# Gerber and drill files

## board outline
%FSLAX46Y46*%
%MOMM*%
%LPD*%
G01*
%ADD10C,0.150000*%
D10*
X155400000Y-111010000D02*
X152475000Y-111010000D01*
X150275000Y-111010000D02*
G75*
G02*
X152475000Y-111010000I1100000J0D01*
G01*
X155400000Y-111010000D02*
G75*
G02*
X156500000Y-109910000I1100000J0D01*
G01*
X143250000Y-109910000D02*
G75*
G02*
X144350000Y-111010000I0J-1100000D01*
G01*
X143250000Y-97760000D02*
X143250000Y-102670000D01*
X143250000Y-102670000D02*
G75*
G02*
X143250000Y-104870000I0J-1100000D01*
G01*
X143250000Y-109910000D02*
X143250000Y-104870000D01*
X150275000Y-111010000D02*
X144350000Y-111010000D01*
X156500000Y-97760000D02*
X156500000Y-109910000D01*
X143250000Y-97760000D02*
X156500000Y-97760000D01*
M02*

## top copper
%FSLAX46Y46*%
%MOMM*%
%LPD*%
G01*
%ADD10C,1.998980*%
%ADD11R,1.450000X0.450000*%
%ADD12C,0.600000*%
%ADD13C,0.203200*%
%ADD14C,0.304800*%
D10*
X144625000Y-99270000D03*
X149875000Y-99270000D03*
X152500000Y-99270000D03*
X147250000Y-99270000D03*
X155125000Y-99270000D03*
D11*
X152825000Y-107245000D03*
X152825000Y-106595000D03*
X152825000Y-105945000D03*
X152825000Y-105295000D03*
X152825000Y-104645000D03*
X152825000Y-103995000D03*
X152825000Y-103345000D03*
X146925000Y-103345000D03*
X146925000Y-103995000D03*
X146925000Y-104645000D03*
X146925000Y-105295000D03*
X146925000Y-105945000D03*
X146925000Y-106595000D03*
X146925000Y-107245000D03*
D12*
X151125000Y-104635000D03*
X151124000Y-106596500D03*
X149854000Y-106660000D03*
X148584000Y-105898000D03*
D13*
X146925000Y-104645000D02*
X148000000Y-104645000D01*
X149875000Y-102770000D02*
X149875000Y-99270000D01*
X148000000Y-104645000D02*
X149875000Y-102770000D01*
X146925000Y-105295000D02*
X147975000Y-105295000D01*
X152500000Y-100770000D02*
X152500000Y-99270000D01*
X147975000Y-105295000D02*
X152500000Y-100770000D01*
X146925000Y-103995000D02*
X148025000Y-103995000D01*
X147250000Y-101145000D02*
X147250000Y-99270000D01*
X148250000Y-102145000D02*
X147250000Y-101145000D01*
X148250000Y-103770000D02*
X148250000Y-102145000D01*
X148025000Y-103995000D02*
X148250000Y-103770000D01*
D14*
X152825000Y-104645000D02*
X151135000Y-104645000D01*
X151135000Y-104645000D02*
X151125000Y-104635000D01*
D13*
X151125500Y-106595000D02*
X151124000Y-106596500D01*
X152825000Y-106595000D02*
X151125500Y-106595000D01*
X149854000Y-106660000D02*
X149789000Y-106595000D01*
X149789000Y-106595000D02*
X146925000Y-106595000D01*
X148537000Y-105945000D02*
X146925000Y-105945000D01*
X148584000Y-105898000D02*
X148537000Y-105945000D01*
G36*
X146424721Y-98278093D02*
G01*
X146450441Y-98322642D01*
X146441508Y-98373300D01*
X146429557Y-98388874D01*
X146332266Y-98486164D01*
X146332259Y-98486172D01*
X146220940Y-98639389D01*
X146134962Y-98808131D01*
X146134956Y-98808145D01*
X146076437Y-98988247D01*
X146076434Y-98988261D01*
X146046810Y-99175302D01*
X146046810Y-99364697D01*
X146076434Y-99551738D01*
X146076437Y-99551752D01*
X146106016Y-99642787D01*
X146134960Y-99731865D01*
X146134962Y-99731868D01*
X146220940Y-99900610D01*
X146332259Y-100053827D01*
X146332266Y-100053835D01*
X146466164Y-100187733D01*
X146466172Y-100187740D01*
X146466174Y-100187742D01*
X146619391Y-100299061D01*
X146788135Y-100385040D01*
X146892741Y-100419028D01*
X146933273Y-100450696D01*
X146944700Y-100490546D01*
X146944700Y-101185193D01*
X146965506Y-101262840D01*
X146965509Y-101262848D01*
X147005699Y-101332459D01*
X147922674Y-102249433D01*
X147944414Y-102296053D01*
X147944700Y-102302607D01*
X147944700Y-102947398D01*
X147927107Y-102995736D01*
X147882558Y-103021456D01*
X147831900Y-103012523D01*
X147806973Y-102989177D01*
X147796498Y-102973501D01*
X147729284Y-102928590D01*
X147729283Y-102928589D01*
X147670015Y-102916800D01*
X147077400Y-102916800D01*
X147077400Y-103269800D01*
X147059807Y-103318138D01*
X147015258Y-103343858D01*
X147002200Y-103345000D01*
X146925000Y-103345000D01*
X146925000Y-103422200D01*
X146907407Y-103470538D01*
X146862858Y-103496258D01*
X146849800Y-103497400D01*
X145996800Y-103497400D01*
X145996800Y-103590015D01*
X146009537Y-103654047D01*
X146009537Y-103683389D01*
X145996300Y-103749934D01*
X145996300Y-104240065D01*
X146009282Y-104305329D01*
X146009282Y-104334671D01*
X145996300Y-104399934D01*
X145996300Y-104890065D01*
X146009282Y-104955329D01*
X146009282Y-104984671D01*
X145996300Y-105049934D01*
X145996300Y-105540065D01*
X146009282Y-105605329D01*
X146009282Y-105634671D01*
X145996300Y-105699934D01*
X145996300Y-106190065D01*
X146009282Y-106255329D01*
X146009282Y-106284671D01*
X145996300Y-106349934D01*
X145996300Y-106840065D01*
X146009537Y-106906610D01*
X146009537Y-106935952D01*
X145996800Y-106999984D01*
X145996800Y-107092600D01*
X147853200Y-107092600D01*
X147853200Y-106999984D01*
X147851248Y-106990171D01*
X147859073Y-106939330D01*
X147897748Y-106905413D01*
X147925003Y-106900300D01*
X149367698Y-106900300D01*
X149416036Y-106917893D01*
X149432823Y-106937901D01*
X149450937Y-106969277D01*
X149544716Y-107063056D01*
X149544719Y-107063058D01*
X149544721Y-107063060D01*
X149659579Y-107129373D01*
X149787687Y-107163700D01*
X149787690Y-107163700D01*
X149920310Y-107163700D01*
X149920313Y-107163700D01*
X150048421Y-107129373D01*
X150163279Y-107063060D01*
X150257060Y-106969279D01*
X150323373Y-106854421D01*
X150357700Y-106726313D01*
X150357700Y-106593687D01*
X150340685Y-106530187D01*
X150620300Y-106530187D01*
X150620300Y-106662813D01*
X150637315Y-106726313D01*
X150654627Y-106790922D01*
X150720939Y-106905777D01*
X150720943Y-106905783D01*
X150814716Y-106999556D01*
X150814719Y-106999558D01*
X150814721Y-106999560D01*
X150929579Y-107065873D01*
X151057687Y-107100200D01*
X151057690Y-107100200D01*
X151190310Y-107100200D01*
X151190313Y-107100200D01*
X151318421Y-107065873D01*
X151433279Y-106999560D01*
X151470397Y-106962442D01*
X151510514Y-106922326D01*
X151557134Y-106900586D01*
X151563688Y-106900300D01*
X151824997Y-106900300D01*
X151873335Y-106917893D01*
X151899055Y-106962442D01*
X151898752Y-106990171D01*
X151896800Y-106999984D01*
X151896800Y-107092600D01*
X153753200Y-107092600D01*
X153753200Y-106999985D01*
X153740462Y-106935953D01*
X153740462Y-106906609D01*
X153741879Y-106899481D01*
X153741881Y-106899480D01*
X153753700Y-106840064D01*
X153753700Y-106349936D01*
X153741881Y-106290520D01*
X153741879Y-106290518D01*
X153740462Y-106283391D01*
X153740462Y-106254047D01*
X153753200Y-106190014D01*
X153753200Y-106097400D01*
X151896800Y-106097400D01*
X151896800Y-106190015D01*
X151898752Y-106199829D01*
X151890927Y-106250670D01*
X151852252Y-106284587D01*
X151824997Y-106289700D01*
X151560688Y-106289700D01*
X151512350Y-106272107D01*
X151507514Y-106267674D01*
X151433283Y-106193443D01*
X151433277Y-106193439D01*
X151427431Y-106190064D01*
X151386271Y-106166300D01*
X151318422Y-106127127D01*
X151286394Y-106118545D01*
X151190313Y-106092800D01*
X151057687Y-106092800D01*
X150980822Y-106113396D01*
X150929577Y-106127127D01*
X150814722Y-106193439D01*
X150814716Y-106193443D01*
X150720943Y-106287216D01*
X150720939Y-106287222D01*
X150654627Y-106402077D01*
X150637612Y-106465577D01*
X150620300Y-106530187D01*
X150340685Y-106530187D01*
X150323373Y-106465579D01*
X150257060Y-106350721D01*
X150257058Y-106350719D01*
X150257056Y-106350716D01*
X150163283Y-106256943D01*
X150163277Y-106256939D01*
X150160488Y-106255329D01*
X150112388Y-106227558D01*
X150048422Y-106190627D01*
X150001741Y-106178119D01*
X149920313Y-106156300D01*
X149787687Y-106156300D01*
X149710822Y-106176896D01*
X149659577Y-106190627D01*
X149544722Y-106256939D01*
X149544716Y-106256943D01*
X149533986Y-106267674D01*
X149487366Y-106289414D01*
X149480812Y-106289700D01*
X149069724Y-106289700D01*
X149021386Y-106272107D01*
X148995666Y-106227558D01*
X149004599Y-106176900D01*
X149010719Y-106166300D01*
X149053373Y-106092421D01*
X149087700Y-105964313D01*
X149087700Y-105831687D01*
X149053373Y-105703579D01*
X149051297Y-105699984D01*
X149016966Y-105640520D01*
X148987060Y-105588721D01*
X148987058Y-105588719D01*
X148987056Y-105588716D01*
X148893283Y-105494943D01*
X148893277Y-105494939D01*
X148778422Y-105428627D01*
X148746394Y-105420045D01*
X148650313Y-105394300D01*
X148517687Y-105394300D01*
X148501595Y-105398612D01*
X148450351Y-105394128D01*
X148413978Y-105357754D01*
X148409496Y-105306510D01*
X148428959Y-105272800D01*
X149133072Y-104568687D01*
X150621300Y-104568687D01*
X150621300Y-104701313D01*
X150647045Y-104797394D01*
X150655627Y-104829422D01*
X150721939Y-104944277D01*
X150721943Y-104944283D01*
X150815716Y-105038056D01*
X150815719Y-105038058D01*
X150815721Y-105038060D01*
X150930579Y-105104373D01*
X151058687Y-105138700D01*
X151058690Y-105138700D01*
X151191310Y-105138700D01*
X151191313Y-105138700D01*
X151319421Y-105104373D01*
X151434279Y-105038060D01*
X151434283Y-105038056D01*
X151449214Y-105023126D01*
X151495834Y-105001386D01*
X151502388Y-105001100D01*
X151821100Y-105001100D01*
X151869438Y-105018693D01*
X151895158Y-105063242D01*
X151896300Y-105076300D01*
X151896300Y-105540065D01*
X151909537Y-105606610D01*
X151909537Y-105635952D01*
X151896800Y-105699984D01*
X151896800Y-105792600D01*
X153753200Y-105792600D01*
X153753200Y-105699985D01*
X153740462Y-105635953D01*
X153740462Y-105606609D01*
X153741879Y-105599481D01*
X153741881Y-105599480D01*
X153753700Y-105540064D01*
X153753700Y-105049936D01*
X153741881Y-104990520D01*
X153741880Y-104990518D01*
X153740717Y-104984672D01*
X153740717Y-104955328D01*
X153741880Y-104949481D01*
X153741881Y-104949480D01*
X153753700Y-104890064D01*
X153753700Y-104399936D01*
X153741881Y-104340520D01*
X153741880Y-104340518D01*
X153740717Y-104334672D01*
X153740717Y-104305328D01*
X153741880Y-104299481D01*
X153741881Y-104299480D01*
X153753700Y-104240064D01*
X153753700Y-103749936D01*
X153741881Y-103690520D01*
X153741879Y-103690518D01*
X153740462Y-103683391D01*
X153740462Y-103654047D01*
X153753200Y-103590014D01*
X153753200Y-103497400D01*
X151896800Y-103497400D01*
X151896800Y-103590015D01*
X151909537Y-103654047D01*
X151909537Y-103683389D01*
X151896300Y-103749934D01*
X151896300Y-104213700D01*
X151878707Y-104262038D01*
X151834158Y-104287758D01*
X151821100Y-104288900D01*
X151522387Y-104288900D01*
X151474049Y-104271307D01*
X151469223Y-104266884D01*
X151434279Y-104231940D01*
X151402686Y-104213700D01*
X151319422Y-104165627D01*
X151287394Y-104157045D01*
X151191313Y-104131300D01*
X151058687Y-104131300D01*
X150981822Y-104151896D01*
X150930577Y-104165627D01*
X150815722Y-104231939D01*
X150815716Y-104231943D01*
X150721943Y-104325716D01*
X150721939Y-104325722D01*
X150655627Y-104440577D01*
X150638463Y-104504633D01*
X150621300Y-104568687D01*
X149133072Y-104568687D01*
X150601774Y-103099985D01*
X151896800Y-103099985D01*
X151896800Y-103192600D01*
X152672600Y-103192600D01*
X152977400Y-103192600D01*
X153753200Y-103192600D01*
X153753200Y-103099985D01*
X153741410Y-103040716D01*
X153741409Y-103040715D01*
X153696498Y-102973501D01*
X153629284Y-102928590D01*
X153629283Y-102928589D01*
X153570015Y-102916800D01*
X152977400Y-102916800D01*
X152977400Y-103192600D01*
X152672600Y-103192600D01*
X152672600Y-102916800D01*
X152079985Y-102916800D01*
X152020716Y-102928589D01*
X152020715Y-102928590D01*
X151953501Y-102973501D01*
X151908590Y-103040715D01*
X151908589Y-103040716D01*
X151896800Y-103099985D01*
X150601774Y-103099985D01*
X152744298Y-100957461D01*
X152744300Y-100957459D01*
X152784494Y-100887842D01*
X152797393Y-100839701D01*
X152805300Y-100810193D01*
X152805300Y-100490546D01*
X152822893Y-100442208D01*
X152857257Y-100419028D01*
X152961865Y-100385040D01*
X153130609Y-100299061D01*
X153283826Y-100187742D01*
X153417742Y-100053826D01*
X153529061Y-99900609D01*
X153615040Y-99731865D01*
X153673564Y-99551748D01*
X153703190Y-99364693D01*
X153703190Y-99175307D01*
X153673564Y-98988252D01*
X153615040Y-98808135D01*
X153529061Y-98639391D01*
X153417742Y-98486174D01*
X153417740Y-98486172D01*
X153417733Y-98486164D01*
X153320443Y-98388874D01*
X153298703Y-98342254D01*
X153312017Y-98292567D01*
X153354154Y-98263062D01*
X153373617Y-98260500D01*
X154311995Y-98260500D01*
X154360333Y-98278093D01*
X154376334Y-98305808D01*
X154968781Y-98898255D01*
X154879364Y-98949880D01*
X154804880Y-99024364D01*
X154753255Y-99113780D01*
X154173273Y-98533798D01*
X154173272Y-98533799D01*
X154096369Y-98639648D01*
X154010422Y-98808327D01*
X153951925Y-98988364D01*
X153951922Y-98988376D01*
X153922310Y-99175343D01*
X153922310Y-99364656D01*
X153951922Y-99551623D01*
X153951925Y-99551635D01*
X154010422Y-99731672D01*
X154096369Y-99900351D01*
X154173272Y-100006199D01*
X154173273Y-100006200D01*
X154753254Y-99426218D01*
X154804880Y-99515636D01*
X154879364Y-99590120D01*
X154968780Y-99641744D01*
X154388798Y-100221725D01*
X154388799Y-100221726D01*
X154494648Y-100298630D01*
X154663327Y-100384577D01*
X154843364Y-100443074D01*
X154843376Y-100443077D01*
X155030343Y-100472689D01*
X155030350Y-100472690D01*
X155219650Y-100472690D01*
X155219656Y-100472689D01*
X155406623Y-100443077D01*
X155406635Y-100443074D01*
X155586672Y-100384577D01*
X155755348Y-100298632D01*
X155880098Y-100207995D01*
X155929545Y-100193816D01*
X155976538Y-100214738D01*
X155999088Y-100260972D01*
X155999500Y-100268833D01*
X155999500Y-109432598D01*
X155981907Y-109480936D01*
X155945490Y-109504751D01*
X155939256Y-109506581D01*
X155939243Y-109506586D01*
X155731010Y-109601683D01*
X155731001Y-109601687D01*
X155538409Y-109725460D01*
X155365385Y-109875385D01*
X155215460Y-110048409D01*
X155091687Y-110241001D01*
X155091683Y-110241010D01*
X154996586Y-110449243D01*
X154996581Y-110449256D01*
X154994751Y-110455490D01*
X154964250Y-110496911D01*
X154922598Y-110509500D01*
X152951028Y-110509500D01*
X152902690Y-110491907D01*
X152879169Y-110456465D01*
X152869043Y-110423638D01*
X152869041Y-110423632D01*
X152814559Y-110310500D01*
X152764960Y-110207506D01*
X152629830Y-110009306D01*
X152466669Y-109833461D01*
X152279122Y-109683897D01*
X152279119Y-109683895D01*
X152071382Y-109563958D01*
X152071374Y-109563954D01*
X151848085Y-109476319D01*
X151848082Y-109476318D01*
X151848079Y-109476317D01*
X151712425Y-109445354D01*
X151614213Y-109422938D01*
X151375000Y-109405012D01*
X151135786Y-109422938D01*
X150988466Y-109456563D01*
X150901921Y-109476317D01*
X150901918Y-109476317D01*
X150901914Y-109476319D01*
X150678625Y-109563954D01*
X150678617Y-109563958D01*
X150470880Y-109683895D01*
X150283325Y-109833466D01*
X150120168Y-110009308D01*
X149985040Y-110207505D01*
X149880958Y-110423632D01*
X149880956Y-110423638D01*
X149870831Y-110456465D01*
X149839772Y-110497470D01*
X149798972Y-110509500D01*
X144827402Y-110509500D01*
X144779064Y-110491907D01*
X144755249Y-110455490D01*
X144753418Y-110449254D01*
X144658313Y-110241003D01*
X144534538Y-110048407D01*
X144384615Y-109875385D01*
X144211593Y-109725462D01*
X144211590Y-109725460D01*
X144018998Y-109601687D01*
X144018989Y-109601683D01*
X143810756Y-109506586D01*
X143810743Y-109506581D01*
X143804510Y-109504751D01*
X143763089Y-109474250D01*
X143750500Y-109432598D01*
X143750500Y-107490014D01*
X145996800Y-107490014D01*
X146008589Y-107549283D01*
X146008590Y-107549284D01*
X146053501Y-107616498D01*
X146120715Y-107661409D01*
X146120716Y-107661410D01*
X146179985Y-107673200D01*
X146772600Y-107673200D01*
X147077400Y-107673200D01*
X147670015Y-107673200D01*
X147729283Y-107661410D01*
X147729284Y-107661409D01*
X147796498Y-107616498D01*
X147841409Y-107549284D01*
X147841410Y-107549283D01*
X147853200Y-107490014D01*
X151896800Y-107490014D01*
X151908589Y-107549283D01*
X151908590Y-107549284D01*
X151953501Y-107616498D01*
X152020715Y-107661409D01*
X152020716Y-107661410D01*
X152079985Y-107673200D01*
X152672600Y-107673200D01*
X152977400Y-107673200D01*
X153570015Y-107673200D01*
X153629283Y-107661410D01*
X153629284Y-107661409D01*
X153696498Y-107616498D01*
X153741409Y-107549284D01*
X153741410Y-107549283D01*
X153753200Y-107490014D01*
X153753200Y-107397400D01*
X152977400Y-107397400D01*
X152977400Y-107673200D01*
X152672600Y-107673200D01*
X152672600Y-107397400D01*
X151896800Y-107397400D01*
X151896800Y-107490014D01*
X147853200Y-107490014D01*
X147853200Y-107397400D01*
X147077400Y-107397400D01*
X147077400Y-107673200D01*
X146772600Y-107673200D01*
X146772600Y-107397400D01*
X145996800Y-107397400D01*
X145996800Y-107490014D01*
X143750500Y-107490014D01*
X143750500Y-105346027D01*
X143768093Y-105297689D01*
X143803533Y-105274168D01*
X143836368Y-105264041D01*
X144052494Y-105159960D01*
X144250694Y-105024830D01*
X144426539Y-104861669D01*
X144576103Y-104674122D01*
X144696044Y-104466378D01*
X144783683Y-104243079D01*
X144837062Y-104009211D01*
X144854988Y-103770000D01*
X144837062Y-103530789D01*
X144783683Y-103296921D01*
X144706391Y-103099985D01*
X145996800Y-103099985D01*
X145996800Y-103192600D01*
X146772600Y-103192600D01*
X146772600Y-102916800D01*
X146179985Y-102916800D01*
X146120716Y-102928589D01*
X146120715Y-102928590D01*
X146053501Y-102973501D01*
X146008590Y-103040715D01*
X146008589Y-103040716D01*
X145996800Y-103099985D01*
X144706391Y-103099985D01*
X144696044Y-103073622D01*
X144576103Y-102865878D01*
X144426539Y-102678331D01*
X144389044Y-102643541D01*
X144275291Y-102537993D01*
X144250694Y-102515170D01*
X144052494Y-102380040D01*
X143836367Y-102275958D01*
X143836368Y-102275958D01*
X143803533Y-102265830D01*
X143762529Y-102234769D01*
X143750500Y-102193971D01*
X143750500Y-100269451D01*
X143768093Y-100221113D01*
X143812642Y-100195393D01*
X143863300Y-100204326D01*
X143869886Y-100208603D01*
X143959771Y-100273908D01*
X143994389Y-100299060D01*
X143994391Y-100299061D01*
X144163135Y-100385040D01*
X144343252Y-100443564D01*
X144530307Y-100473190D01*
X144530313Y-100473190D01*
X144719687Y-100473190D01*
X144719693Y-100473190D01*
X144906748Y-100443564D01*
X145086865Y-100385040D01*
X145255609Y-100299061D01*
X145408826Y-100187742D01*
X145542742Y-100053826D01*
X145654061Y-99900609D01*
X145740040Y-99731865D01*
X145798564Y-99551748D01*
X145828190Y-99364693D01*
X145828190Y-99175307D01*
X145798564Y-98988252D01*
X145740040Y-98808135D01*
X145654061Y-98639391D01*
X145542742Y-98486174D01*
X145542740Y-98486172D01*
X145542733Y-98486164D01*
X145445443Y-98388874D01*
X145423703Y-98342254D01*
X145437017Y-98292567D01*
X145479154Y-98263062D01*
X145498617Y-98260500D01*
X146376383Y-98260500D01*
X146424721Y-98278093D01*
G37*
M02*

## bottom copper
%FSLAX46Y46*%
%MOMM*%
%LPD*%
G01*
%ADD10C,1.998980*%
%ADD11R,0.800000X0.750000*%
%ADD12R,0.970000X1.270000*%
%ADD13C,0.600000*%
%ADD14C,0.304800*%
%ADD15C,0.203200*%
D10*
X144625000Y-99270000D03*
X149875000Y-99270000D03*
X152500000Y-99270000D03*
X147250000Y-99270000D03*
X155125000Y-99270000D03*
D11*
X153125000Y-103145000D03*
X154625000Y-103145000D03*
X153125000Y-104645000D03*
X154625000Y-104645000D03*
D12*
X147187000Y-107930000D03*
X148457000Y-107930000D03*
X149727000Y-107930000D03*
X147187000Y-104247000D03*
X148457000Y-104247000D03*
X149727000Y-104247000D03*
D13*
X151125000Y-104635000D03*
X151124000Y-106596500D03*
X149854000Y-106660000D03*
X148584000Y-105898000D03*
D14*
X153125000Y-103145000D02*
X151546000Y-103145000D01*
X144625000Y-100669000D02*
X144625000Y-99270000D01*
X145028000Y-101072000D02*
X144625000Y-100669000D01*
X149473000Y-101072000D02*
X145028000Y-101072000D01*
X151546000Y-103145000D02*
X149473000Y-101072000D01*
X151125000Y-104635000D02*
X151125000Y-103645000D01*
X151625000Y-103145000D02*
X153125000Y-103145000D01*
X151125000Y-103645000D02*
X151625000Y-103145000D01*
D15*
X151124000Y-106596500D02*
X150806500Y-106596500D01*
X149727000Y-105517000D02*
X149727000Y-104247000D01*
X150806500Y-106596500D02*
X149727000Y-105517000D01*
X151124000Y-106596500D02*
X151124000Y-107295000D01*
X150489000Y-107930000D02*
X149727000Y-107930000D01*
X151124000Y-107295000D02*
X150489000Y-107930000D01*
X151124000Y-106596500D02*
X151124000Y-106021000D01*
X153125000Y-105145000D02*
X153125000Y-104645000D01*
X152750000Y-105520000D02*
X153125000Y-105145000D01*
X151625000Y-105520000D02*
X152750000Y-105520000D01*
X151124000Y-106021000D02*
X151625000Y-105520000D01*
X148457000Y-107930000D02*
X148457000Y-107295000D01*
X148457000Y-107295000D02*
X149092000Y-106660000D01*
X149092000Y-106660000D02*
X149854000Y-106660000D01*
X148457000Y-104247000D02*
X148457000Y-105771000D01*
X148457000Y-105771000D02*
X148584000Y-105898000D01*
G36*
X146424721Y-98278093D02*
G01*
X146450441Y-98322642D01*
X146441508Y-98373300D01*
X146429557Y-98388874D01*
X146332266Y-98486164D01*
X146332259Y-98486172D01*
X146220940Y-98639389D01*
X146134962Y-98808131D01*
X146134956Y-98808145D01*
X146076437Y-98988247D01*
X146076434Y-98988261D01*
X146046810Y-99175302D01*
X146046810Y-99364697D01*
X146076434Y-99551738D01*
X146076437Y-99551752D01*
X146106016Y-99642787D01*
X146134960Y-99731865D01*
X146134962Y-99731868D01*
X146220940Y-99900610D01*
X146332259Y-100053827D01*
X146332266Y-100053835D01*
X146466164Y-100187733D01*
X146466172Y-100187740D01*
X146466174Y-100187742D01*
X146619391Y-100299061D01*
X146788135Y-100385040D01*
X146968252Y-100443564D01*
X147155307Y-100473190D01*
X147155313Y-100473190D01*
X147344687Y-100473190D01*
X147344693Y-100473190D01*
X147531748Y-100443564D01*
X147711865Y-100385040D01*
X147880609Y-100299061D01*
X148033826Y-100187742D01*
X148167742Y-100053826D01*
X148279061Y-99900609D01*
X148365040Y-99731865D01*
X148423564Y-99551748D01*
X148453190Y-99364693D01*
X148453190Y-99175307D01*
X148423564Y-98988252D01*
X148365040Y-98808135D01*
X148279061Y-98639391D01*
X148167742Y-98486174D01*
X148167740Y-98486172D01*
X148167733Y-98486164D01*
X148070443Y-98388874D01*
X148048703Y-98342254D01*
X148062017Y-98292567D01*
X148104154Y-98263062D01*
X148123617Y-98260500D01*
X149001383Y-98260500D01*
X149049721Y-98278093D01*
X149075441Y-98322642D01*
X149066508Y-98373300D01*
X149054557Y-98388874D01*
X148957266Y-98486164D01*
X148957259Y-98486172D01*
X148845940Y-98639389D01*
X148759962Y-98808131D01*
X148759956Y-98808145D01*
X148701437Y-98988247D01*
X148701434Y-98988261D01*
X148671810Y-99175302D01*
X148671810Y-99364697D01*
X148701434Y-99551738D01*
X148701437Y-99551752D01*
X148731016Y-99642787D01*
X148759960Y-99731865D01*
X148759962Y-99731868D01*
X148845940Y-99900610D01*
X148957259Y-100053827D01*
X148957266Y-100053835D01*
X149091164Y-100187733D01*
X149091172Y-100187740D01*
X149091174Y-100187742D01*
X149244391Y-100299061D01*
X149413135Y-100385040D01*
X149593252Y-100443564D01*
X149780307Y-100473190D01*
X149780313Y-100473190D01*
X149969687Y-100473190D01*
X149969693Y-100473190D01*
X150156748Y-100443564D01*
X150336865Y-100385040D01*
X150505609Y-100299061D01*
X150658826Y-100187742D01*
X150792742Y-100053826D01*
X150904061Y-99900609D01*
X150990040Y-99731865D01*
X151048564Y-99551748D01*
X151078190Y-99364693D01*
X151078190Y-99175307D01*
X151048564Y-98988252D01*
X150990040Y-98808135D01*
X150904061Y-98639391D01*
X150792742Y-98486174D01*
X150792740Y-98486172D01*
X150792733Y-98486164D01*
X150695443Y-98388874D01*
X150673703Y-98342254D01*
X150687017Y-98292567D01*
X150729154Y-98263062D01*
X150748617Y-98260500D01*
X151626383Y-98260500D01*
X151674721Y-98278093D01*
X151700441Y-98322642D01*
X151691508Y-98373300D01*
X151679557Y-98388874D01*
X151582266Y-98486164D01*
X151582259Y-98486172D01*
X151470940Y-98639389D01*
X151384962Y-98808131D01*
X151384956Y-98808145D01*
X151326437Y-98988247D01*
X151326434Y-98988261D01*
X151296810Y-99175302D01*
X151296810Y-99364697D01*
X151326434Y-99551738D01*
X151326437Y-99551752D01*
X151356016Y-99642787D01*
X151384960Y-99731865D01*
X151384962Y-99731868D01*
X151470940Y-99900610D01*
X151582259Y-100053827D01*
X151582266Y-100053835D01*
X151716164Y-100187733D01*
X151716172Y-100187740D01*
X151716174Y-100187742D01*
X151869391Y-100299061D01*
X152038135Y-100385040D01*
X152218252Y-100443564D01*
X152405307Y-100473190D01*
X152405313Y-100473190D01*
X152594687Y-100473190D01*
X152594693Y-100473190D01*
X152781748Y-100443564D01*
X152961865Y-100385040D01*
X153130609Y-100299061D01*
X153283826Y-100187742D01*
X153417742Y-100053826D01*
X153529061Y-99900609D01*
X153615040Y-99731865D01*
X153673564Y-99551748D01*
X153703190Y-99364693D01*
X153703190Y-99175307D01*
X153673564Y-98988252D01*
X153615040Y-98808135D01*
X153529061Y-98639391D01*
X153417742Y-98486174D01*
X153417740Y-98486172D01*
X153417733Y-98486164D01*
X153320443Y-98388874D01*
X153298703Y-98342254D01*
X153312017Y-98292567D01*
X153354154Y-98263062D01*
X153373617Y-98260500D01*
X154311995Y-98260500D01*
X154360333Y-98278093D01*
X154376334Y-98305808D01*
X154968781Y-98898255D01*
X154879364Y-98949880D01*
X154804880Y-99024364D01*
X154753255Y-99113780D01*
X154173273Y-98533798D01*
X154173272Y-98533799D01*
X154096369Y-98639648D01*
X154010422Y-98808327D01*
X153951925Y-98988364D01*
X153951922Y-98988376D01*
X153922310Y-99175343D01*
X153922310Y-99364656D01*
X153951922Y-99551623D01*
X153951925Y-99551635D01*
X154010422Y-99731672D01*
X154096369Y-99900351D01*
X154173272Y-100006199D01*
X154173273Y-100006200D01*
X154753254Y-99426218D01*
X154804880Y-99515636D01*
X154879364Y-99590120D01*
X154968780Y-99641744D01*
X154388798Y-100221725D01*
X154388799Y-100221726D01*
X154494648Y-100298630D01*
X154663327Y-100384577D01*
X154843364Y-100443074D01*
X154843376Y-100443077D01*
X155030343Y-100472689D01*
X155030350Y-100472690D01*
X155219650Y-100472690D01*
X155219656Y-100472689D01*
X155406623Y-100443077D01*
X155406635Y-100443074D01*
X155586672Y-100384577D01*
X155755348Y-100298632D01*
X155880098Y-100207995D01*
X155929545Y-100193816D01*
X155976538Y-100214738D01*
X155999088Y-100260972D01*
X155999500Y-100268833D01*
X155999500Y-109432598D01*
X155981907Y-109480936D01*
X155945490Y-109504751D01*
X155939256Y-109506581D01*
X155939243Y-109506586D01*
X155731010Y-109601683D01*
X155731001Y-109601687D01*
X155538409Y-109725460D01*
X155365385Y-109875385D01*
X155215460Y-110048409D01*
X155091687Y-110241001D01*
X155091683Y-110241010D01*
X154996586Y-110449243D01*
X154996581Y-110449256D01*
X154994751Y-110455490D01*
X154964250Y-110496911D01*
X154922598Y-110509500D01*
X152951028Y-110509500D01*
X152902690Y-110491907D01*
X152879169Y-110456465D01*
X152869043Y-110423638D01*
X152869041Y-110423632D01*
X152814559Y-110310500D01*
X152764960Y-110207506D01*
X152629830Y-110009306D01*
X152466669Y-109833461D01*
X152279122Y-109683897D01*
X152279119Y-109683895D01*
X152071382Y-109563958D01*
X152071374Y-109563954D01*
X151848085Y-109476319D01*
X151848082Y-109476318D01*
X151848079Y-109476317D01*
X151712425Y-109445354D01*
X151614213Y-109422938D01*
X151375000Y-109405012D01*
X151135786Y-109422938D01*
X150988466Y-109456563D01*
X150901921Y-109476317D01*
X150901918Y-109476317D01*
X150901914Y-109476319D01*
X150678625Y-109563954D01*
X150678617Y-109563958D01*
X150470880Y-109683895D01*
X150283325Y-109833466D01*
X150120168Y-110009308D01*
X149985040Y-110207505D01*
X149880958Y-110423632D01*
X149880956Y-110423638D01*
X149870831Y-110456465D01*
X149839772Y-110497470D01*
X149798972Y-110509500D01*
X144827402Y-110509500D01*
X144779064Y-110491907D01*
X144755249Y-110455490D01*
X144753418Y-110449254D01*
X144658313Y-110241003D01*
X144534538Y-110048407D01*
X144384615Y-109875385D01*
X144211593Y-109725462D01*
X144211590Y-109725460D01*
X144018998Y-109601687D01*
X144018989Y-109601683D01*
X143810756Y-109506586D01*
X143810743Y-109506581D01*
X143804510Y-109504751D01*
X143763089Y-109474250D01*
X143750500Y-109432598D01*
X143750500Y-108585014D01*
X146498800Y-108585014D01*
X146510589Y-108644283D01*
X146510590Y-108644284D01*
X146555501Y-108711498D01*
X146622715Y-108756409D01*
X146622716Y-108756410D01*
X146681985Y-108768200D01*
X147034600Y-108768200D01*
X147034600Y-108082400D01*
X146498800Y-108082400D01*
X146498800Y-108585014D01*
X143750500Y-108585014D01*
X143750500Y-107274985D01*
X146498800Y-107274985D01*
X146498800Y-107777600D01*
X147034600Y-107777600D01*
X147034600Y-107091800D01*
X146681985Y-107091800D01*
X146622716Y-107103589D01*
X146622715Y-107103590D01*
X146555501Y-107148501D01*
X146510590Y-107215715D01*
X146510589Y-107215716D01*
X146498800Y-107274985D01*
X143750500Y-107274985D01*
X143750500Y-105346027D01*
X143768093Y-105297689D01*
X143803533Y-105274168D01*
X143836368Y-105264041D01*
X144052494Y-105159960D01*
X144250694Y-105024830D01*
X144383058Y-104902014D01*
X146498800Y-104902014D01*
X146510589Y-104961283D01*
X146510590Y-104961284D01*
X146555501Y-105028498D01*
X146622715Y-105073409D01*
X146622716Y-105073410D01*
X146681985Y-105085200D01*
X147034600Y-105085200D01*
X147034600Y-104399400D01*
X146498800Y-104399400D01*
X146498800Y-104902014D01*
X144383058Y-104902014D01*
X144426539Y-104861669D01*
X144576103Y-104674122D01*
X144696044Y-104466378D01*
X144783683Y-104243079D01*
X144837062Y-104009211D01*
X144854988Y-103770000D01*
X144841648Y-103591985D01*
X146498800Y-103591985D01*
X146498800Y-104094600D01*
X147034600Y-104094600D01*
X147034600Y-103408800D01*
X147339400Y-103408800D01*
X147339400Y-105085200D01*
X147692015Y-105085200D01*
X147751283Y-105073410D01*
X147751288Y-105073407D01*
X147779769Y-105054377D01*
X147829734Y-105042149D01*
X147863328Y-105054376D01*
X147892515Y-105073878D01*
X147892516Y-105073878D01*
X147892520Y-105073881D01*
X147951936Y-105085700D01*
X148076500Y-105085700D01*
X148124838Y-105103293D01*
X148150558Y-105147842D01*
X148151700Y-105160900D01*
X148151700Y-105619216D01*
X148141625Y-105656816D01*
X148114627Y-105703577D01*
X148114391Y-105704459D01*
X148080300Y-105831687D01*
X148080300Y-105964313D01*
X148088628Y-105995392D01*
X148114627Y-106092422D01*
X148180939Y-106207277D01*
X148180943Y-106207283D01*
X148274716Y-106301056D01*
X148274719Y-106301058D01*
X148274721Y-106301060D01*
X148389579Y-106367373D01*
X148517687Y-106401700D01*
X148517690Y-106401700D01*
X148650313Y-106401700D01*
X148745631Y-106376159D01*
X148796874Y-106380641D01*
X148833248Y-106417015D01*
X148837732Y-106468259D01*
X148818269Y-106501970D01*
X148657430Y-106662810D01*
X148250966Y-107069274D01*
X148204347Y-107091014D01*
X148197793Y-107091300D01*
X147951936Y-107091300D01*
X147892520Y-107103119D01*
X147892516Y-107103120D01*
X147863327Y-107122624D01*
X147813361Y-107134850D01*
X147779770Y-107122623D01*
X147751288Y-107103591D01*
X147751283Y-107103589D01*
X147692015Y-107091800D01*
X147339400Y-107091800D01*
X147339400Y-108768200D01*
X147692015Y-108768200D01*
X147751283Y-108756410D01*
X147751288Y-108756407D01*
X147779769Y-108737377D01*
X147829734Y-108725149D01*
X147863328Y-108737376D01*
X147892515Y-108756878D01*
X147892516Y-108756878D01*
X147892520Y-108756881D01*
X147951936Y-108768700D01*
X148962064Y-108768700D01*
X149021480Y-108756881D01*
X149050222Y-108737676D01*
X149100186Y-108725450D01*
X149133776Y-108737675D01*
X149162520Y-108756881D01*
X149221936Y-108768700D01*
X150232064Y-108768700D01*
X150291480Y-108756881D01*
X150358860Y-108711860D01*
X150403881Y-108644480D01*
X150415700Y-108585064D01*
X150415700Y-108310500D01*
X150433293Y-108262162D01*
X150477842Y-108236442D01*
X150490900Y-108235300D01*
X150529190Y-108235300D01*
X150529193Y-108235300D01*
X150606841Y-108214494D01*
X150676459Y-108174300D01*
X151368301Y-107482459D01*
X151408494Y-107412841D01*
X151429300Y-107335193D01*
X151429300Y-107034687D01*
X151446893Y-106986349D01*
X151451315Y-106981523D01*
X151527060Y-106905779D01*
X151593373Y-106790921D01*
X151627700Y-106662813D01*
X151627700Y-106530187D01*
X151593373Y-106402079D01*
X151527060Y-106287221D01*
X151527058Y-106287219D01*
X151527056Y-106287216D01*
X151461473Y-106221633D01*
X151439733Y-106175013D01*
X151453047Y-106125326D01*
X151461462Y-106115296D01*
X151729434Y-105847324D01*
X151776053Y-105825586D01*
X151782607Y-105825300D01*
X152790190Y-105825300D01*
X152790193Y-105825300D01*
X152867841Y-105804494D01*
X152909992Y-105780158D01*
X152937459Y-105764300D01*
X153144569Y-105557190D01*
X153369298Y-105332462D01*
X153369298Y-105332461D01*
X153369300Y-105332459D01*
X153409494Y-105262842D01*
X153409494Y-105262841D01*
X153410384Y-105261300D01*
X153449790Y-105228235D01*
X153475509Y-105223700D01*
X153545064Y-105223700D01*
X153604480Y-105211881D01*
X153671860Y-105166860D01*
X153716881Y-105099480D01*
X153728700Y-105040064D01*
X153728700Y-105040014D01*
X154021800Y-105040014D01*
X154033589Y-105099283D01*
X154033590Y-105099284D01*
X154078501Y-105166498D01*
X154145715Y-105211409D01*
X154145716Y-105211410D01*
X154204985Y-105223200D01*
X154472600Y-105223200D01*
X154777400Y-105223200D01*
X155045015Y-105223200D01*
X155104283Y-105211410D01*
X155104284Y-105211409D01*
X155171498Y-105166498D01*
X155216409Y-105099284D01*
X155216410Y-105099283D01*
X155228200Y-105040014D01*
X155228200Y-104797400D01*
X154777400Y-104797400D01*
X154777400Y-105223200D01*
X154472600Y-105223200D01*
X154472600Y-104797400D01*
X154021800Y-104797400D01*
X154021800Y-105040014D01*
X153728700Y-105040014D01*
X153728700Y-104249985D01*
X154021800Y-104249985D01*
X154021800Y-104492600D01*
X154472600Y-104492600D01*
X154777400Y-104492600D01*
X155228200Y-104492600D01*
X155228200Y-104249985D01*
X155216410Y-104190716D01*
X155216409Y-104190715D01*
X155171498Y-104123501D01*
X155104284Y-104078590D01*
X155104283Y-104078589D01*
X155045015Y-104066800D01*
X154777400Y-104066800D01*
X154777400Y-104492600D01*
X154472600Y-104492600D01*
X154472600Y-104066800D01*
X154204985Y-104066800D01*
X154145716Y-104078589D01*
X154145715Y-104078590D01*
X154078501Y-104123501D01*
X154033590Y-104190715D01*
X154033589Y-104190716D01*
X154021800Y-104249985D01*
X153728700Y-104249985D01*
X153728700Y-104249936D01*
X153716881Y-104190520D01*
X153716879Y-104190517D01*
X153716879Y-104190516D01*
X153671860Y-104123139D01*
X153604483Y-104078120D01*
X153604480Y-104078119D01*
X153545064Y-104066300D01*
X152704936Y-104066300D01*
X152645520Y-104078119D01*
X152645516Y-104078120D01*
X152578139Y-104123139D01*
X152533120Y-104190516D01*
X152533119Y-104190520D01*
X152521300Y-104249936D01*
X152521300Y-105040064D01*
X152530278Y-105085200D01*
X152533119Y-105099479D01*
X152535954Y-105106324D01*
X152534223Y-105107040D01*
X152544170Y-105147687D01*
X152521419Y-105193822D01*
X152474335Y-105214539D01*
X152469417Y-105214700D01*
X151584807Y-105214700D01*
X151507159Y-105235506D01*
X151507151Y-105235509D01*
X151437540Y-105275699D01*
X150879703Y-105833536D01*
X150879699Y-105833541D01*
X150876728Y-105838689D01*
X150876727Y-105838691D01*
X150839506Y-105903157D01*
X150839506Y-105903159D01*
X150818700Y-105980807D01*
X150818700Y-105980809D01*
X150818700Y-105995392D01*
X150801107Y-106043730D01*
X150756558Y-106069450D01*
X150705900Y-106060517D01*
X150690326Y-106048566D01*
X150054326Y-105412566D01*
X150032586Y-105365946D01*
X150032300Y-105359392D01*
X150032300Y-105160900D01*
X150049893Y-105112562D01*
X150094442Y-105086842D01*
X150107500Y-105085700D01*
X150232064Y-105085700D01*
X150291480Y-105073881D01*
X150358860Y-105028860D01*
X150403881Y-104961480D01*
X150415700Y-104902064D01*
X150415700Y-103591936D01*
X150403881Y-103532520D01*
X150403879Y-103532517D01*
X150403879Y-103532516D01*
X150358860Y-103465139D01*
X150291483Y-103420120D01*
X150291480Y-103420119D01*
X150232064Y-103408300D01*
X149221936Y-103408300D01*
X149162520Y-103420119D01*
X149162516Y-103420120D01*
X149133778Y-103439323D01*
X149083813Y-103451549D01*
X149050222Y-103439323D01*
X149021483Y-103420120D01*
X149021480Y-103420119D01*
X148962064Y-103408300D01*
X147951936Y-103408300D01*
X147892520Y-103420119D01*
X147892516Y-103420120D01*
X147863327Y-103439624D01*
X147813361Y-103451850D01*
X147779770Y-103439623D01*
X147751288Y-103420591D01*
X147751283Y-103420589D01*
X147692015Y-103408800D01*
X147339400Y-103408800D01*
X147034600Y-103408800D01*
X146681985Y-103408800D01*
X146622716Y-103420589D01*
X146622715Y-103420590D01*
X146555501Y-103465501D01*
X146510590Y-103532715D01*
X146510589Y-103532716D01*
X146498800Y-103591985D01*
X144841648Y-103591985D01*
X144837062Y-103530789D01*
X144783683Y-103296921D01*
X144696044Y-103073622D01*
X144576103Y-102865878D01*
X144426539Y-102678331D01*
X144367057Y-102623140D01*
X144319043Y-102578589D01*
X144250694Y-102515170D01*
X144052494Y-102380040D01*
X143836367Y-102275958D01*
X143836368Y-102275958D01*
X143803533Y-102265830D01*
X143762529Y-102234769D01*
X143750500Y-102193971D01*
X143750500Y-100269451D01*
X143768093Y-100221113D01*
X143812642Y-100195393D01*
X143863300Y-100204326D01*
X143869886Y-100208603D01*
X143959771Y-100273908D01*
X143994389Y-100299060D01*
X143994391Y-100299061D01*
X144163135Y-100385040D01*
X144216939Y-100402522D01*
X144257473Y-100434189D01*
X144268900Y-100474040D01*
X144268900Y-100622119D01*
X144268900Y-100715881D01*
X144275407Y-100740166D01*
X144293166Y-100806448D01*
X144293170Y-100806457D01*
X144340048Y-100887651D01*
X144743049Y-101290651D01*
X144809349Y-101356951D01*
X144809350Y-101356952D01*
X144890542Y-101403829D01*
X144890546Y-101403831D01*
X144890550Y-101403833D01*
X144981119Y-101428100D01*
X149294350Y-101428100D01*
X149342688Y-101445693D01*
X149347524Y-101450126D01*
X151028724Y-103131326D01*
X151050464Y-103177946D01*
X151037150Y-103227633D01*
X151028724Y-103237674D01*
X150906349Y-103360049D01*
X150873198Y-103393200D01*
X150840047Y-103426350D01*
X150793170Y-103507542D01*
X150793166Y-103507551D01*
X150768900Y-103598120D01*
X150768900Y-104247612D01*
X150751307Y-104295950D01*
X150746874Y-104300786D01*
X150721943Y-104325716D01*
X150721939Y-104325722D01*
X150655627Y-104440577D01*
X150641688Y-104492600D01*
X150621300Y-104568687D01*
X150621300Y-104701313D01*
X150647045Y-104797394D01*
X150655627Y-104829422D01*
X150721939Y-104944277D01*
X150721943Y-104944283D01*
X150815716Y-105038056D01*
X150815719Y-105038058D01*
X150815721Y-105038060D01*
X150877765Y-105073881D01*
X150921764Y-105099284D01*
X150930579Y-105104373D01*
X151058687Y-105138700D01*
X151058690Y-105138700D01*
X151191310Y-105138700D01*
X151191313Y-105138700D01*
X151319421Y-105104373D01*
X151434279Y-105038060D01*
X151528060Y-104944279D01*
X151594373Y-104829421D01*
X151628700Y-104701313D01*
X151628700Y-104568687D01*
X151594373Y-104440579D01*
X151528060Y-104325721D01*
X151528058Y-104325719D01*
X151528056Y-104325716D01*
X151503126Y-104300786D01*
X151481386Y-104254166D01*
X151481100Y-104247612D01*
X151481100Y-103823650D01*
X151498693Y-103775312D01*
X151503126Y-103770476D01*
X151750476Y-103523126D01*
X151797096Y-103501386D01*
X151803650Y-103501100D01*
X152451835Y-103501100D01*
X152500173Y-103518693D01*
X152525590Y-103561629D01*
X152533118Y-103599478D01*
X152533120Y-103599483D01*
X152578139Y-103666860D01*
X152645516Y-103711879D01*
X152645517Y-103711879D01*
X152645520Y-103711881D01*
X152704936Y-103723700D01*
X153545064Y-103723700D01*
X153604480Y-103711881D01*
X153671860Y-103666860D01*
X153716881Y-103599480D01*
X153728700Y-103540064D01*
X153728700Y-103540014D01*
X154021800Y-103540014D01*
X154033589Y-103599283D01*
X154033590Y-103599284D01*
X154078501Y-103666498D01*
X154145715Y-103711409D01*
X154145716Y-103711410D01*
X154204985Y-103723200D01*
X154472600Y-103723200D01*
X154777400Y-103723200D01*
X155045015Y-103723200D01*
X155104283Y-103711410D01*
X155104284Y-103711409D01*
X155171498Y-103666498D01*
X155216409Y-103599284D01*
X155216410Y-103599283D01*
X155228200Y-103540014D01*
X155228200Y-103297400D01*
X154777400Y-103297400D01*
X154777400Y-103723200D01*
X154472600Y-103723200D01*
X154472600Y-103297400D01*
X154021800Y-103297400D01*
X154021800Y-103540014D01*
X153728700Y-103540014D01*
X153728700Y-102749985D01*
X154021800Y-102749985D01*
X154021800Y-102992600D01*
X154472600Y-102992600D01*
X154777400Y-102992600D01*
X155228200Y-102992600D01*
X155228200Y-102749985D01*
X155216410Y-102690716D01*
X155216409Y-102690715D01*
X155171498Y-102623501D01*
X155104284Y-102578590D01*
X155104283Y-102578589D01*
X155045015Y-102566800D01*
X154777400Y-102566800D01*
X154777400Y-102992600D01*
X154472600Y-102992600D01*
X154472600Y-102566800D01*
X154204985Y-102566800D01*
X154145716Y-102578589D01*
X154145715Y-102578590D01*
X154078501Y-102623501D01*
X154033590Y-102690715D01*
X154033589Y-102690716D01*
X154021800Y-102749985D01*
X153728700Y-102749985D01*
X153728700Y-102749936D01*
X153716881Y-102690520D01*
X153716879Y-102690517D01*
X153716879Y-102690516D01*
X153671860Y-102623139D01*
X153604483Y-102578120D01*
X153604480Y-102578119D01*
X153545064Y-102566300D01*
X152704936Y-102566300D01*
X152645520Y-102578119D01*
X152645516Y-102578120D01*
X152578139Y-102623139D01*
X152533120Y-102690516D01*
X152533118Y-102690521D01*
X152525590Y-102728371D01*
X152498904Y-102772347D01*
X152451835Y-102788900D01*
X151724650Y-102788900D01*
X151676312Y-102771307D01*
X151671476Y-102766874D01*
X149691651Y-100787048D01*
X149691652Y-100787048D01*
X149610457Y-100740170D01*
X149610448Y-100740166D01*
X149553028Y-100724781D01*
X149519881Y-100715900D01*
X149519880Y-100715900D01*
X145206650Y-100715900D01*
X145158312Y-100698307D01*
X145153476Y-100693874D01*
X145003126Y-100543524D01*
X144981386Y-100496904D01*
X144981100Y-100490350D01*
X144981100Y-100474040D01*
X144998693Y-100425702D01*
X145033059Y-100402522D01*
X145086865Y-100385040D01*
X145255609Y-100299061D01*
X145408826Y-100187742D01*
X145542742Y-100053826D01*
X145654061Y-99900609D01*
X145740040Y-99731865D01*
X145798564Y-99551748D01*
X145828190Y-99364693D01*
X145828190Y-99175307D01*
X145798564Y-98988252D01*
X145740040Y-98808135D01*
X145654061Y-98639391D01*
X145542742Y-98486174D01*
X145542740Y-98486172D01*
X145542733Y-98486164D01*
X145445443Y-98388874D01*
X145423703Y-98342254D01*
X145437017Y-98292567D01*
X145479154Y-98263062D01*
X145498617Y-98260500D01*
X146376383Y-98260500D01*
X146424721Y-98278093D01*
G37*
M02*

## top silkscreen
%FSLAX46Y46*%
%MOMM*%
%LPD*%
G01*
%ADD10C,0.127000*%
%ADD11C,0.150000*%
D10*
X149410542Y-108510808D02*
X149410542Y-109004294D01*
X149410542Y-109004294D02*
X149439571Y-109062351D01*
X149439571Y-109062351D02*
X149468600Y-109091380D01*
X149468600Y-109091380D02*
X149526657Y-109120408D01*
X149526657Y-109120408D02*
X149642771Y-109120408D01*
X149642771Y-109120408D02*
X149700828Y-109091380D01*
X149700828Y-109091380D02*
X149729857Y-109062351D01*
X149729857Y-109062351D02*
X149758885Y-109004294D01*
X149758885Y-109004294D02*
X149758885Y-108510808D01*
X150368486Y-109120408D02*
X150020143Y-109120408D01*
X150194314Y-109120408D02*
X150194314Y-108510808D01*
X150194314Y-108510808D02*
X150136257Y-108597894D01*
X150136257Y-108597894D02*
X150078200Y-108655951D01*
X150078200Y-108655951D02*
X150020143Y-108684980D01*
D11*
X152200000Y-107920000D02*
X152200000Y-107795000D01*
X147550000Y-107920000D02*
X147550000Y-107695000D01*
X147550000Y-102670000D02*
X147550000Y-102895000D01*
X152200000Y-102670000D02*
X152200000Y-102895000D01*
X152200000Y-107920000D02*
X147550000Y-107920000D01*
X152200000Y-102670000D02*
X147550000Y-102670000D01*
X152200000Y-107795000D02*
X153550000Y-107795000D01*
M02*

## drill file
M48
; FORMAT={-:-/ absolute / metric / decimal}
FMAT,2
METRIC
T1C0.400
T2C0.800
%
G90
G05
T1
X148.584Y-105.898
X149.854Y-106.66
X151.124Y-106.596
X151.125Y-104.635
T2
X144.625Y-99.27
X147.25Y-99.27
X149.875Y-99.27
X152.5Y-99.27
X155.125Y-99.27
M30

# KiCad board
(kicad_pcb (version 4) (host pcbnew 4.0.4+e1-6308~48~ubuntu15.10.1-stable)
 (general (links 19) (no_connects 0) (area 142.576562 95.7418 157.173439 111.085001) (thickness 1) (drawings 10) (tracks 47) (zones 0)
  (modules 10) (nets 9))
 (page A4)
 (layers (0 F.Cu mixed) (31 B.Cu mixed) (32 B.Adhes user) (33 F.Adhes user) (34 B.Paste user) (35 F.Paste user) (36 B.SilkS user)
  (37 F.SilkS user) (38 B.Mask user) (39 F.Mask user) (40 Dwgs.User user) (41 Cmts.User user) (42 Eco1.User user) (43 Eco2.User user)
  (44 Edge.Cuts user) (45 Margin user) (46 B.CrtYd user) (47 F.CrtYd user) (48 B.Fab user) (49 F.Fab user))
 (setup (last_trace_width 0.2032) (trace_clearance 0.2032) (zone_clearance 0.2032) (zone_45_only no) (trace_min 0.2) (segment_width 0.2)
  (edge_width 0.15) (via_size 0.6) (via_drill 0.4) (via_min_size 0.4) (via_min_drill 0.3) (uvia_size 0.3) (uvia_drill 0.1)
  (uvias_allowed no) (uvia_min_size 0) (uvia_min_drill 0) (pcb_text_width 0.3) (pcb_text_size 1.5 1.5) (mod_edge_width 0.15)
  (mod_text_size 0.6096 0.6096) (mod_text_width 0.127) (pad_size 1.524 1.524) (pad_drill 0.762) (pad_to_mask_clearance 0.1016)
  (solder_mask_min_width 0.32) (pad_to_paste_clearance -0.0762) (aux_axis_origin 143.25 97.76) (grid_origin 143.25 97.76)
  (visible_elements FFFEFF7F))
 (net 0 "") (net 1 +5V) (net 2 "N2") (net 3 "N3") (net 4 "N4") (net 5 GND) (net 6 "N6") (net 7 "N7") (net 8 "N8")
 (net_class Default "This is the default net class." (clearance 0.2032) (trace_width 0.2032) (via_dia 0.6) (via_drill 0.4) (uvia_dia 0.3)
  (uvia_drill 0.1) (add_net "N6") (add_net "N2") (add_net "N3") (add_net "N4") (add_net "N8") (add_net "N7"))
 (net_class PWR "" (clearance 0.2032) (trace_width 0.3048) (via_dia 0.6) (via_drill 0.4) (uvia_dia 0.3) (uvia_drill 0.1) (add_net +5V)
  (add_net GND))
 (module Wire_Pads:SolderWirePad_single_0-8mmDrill (layer B.Cu) (at 144.625 99.27)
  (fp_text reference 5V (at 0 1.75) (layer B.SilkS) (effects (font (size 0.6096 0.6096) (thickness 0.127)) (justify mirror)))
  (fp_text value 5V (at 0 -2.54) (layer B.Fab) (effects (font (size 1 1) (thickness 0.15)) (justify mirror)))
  (pad 1 thru_hole circle (at 0 0) (size 1.99898 1.99898) (drill 0.8001) (layers *.Cu *.Mask) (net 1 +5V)))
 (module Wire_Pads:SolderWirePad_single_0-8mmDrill (layer B.Cu) (at 149.875 99.27)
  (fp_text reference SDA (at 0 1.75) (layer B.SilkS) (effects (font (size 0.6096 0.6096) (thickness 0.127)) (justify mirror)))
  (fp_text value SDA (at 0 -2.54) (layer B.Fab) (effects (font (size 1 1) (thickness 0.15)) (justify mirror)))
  (pad 1 thru_hole circle (at 0 0) (size 1.99898 1.99898) (drill 0.8001) (layers *.Cu *.Mask) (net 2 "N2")))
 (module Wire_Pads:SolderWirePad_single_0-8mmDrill (layer B.Cu) (at 152.5 99.27)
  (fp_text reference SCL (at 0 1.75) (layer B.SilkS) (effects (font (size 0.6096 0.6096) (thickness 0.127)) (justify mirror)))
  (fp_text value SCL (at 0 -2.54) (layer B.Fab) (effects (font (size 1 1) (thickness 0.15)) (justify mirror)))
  (pad 1 thru_hole circle (at 0 0) (size 1.99898 1.99898) (drill 0.8001) (layers *.Cu *.Mask) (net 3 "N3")))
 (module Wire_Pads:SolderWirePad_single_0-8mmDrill (layer B.Cu) (at 147.25 99.27)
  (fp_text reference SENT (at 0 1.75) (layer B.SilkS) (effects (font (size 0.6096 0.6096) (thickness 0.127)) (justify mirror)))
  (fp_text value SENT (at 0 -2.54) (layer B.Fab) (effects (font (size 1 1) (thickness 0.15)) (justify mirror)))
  (pad 1 thru_hole circle (at 0 0) (size 1.99898 1.99898) (drill 0.8001) (layers *.Cu *.Mask) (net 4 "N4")))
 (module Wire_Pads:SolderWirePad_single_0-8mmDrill (layer B.Cu) (at 155.125 99.27)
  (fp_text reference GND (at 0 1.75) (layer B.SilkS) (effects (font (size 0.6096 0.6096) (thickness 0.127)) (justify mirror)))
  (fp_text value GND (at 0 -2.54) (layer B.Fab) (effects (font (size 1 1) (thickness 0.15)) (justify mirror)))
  (pad 1 thru_hole circle (at 0 0) (size 1.99898 1.99898) (drill 0.8001) (layers *.Cu *.Mask) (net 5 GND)))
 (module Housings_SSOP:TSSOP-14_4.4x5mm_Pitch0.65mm (layer F.Cu) (at 149.875 105.295 180)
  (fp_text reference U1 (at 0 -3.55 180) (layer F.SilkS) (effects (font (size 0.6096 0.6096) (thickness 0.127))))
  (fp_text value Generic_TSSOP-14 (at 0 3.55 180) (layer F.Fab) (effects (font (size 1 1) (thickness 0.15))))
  (fp_line (start -2.325 -2.625) (end -2.325 -2.5) (layer F.SilkS) (width 0.15))
  (fp_line (start 2.325 -2.625) (end 2.325 -2.4) (layer F.SilkS) (width 0.15))
  (fp_line (start 2.325 2.625) (end 2.325 2.4) (layer F.SilkS) (width 0.15))
  (fp_line (start -2.325 2.625) (end -2.325 2.4) (layer F.SilkS) (width 0.15))
  (fp_line (start -2.325 -2.625) (end 2.325 -2.625) (layer F.SilkS) (width 0.15))
  (fp_line (start -2.325 2.625) (end 2.325 2.625) (layer F.SilkS) (width 0.15))
  (fp_line (start -2.325 -2.5) (end -3.675 -2.5) (layer F.SilkS) (width 0.15))
  (pad 1 smd rect (at -2.95 -1.95 180) (size 1.45 0.45) (layers F.Cu F.Paste F.Mask) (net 5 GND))
  (pad 2 smd rect (at -2.95 -1.3 180) (size 1.45 0.45) (layers F.Cu F.Paste F.Mask) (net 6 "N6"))
  (pad 3 smd rect (at -2.95 -0.65 180) (size 1.45 0.45) (layers F.Cu F.Paste F.Mask) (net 5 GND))
  (pad 4 smd rect (at -2.95 0 180) (size 1.45 0.45) (layers F.Cu F.Paste F.Mask))
  (pad 5 smd rect (at -2.95 0.65 180) (size 1.45 0.45) (layers F.Cu F.Paste F.Mask) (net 1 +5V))
  (pad 6 smd rect (at -2.95 1.3 180) (size 1.45 0.45) (layers F.Cu F.Paste F.Mask))
  (pad 7 smd rect (at -2.95 1.95 180) (size 1.45 0.45) (layers F.Cu F.Paste F.Mask) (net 5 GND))
  (pad 8 smd rect (at 2.95 1.95 180) (size 1.45 0.45) (layers F.Cu F.Paste F.Mask) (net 5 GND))
  (pad 9 smd rect (at 2.95 1.3 180) (size 1.45 0.45) (layers F.Cu F.Paste F.Mask) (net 4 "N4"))
  (pad 10 smd rect (at 2.95 0.65 180) (size 1.45 0.45) (layers F.Cu F.Paste F.Mask) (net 2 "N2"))
  (pad 11 smd rect (at 2.95 0 180) (size 1.45 0.45) (layers F.Cu F.Paste F.Mask) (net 3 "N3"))
  (pad 12 smd rect (at 2.95 -0.65 180) (size 1.45 0.45) (layers F.Cu F.Paste F.Mask) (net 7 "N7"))
  (pad 13 smd rect (at 2.95 -1.3 180) (size 1.45 0.45) (layers F.Cu F.Paste F.Mask) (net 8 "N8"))
  (pad 14 smd rect (at 2.95 -1.95 180) (size 1.45 0.45) (layers F.Cu F.Paste F.Mask) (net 5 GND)))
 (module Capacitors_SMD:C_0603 (layer B.Cu) (at 153.875 103.145)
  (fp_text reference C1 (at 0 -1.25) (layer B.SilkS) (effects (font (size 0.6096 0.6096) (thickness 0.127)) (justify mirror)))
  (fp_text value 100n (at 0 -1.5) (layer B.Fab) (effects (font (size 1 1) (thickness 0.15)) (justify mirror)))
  (pad 1 smd rect (at -0.75 0) (size 0.8 0.75) (layers B.Cu B.Paste B.Mask) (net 1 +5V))
  (pad 2 smd rect (at 0.75 0) (size 0.8 0.75) (layers B.Cu B.Paste B.Mask) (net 5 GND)))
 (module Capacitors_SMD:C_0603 (layer B.Cu) (at 153.875 104.645)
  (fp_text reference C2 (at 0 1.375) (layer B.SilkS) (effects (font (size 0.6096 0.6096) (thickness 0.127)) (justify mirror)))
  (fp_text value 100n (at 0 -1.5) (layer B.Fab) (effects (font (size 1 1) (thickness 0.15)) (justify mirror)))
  (pad 1 smd rect (at -0.75 0) (size 0.8 0.75) (layers B.Cu B.Paste B.Mask) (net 6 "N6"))
  (pad 2 smd rect (at 0.75 0) (size 0.8 0.75) (layers B.Cu B.Paste B.Mask) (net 5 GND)))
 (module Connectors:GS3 (layer B.Cu) (at 148.457 107.93 270)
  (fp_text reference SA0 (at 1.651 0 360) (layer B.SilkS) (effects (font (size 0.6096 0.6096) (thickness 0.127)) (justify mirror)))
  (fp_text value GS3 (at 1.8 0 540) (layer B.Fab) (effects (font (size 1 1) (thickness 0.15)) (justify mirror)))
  (pad 1 smd rect (at 0 1.27 270) (size 1.27 0.97) (layers B.Cu B.Paste B.Mask) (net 5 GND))
  (pad 2 smd rect (at 0 0 270) (size 1.27 0.97) (layers B.Cu B.Paste B.Mask) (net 8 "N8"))
  (pad 3 smd rect (at 0 -1.27 270) (size 1.27 0.97) (layers B.Cu B.Paste B.Mask) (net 6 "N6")))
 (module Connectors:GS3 (layer B.Cu) (at 148.457 104.247 270)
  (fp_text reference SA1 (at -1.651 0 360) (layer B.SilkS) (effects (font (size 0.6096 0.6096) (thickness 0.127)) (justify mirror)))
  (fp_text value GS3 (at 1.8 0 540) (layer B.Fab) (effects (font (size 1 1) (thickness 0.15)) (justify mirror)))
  (pad 1 smd rect (at 0 1.27 270) (size 1.27 0.97) (layers B.Cu B.Paste B.Mask) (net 5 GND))
  (pad 2 smd rect (at 0 0 270) (size 1.27 0.97) (layers B.Cu B.Paste B.Mask) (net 7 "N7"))
  (pad 3 smd rect (at 0 -1.27 270) (size 1.27 0.97) (layers B.Cu B.Paste B.Mask) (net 6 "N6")))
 (gr_line (start 155.4 111.01) (end 152.475 111.01) (angle 90) (layer Edge.Cuts) (width 0.15))
 (gr_arc (start 151.375 111.01) (end 150.275 111.01) (angle 180) (layer Edge.Cuts) (width 0.15))
 (gr_arc (start 156.5 111.01) (end 155.4 111.01) (angle 90) (layer Edge.Cuts) (width 0.15))
 (gr_arc (start 143.25 111.01) (end 143.25 109.91) (angle 90) (layer Edge.Cuts) (width 0.15))
 (gr_line (start 143.25 97.76) (end 143.25 102.67) (angle 90) (layer Edge.Cuts) (width 0.15))
 (gr_arc (start 143.25 103.77) (end 143.25 102.67) (angle 180) (layer Edge.Cuts) (width 0.15))
 (gr_line (start 143.25 109.91) (end 143.25 104.87) (angle 90) (layer Edge.Cuts) (width 0.15))
 (gr_line (start 150.275 111.01) (end 144.35 111.01) (angle 90) (layer Edge.Cuts) (width 0.15))
 (gr_line (start 156.5 97.76) (end 156.5 109.91) (angle 90) (layer Edge.Cuts) (width 0.15))
 (gr_line (start 143.25 97.76) (end 156.5 97.76) (angle 90) (layer Edge.Cuts) (width 0.15))
 (segment (start 146.925 104.645) (end 148 104.645) (width 0.2032) (layer F.Cu) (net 2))
 (segment (start 149.875 102.77) (end 149.875 99.27) (width 0.2032) (layer F.Cu) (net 2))
 (segment (start 148 104.645) (end 149.875 102.77) (width 0.2032) (layer F.Cu) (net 2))
 (segment (start 146.925 105.295) (end 147.975 105.295) (width 0.2032) (layer F.Cu) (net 3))
 (segment (start 152.5 100.77) (end 152.5 99.27) (width 0.2032) (layer F.Cu) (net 3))
 (segment (start 147.975 105.295) (end 152.5 100.77) (width 0.2032) (layer F.Cu) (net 3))
 (segment (start 146.925 103.995) (end 148.025 103.995) (width 0.2032) (layer F.Cu) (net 4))
 (segment (start 147.25 101.145) (end 147.25 99.27) (width 0.2032) (layer F.Cu) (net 4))
 (segment (start 148.25 102.145) (end 147.25 101.145) (width 0.2032) (layer F.Cu) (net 4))
 (segment (start 148.25 103.77) (end 148.25 102.145) (width 0.2032) (layer F.Cu) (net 4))
 (segment (start 148.025 103.995) (end 148.25 103.77) (width 0.2032) (layer F.Cu) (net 4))
 (segment (start 153.125 103.145) (end 151.546 103.145) (width 0.3048) (layer B.Cu) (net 1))
 (segment (start 144.625 100.669) (end 144.625 99.27) (width 0.3048) (layer B.Cu) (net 1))
 (segment (start 145.028 101.072) (end 144.625 100.669) (width 0.3048) (layer B.Cu) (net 1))
 (segment (start 149.473 101.072) (end 145.028 101.072) (width 0.3048) (layer B.Cu) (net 1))
 (segment (start 151.546 103.145) (end 149.473 101.072) (width 0.3048) (layer B.Cu) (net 1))
 (segment (start 151.125 104.635) (end 151.125 103.645) (width 0.3048) (layer B.Cu) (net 1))
 (segment (start 152.825 104.645) (end 151.135 104.645) (width 0.3048) (layer F.Cu) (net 1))
 (segment (start 151.135 104.645) (end 151.125 104.635) (width 0.3048) (layer F.Cu) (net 1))
 (via (at 151.125 104.635) (size 0.6) (drill 0.4) (layers F.Cu B.Cu) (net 1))
 (segment (start 151.625 103.145) (end 153.125 103.145) (width 0.3048) (layer B.Cu) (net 1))
 (segment (start 151.125 103.645) (end 151.625 103.145) (width 0.3048) (layer B.Cu) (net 1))
 (segment (start 151.124 106.5965) (end 150.8065 106.5965) (width 0.2032) (layer B.Cu) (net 6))
 (segment (start 149.727 105.517) (end 149.727 104.247) (width 0.2032) (layer B.Cu) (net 6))
 (segment (start 150.8065 106.5965) (end 149.727 105.517) (width 0.2032) (layer B.Cu) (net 6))
 (segment (start 151.124 106.5965) (end 151.124 107.295) (width 0.2032) (layer B.Cu) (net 6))
 (segment (start 150.489 107.93) (end 149.727 107.93) (width 0.2032) (layer B.Cu) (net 6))
 (segment (start 151.124 107.295) (end 150.489 107.93) (width 0.2032) (layer B.Cu) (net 6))
 (segment (start 151.124 106.5965) (end 151.124 106.021) (width 0.2032) (layer B.Cu) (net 6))
 (segment (start 151.1255 106.595) (end 151.124 106.5965) (width 0.2032) (layer F.Cu) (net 6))
 (via (at 151.124 106.5965) (size 0.6) (drill 0.4) (layers F.Cu B.Cu) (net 6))
 (segment (start 152.825 106.595) (end 151.1255 106.595) (width 0.2032) (layer F.Cu) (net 6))
 (segment (start 153.125 105.145) (end 153.125 104.645) (width 0.2032) (layer B.Cu) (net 6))
 (segment (start 152.75 105.52) (end 153.125 105.145) (width 0.2032) (layer B.Cu) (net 6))
 (segment (start 151.625 105.52) (end 152.75 105.52) (width 0.2032) (layer B.Cu) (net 6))
 (segment (start 151.124 106.021) (end 151.625 105.52) (width 0.2032) (layer B.Cu) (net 6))
 (segment (start 148.457 107.93) (end 148.457 107.295) (width 0.2032) (layer B.Cu) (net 8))
 (segment (start 148.457 107.295) (end 149.092 106.66) (width 0.2032) (layer B.Cu) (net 8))
 (segment (start 149.092 106.66) (end 149.854 106.66) (width 0.2032) (layer B.Cu) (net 8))
 (via (at 149.854 106.66) (size 0.6) (drill 0.4) (layers F.Cu B.Cu) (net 8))
 (segment (start 149.854 106.66) (end 149.789 106.595) (width 0.2032) (layer F.Cu) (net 8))
 (segment (start 149.789 106.595) (end 146.925 106.595) (width 0.2032) (layer F.Cu) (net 8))
 (segment (start 148.457 104.247) (end 148.457 105.771) (width 0.2032) (layer B.Cu) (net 7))
 (segment (start 148.537 105.945) (end 146.925 105.945) (width 0.2032) (layer F.Cu) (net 7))
 (segment (start 148.584 105.898) (end 148.537 105.945) (width 0.2032) (layer F.Cu) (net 7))
 (via (at 148.584 105.898) (size 0.6) (drill 0.4) (layers F.Cu B.Cu) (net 7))
 (segment (start 148.457 105.771) (end 148.584 105.898) (width 0.2032) (layer B.Cu) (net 7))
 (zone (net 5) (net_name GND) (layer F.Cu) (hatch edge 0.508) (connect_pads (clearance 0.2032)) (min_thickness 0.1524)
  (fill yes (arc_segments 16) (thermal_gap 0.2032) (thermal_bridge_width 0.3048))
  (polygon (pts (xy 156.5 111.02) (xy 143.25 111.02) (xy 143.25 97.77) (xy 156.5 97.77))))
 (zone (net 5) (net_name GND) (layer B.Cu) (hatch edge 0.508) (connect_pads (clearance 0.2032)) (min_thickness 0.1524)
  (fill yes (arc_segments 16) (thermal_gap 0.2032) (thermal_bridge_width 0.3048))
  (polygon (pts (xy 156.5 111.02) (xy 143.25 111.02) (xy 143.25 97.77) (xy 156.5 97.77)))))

